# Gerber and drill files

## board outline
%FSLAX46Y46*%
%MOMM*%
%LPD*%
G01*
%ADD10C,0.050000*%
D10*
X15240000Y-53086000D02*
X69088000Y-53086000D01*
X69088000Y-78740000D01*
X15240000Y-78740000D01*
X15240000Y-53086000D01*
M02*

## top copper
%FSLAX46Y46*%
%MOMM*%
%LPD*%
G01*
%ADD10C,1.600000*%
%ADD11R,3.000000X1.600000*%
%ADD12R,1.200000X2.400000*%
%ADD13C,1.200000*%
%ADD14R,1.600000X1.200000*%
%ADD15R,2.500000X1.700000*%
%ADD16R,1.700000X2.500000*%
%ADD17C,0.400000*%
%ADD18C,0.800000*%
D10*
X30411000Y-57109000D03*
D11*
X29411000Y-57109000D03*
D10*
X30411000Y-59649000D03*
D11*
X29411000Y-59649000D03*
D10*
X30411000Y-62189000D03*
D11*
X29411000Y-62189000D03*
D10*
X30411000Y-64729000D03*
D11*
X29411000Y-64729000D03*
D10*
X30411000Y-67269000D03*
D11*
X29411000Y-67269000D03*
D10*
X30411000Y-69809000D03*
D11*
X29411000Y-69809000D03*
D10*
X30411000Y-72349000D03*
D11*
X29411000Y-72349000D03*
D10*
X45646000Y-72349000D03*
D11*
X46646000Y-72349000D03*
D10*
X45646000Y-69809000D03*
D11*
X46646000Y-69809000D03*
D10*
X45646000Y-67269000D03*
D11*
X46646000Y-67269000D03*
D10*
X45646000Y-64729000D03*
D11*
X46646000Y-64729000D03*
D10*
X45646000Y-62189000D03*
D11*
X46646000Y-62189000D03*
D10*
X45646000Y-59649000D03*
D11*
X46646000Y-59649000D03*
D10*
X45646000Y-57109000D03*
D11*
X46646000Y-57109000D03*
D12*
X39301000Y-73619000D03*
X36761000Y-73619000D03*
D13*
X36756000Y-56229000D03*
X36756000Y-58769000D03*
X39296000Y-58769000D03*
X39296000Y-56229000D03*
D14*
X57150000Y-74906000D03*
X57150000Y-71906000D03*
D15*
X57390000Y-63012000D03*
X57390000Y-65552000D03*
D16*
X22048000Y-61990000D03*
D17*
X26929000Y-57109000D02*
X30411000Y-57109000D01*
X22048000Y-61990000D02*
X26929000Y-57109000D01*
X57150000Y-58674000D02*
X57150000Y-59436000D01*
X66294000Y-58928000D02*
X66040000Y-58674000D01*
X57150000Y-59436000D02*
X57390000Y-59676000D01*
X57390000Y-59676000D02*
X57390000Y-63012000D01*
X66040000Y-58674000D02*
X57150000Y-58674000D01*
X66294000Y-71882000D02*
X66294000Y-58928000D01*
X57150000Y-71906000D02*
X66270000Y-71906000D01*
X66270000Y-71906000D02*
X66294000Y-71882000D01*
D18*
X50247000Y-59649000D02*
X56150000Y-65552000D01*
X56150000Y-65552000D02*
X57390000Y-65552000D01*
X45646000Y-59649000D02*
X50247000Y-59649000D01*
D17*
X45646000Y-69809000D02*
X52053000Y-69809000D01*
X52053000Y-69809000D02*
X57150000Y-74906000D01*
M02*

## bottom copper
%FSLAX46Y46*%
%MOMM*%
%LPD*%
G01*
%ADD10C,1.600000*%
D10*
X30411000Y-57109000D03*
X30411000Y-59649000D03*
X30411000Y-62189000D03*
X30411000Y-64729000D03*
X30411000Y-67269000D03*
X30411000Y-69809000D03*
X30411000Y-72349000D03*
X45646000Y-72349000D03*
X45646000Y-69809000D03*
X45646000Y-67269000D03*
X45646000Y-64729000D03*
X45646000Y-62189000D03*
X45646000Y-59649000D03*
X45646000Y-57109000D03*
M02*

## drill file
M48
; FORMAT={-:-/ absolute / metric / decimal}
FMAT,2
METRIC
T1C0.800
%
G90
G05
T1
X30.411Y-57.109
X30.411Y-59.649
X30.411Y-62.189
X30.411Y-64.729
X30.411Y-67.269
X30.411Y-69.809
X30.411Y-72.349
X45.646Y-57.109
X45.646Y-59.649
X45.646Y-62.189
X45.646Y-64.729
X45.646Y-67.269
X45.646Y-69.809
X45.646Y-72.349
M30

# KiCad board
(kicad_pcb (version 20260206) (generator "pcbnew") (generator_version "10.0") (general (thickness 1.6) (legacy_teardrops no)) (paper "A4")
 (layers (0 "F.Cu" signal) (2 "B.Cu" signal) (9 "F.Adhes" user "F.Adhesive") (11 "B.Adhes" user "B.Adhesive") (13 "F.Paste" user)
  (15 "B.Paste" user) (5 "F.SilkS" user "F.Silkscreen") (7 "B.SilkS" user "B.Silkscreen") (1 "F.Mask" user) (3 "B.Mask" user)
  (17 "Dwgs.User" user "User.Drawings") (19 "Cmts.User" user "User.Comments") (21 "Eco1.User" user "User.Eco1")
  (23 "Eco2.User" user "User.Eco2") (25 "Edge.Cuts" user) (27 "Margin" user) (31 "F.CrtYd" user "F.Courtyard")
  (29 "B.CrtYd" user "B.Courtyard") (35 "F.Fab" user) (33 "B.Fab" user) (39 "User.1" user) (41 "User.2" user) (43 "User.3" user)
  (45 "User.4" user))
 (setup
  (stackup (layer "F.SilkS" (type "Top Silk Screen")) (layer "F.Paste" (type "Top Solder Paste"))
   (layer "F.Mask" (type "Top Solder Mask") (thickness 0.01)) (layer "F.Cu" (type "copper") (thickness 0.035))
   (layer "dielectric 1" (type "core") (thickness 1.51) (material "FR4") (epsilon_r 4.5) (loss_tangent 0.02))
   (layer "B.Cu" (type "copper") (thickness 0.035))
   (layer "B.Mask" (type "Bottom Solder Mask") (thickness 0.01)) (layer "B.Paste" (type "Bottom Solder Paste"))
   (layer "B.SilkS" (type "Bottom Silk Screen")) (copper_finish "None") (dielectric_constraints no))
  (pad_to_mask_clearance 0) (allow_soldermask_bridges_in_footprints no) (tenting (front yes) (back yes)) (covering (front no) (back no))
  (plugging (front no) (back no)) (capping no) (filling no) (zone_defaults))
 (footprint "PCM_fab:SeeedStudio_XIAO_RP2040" (layer "F.Cu") (at 38.026 64.729)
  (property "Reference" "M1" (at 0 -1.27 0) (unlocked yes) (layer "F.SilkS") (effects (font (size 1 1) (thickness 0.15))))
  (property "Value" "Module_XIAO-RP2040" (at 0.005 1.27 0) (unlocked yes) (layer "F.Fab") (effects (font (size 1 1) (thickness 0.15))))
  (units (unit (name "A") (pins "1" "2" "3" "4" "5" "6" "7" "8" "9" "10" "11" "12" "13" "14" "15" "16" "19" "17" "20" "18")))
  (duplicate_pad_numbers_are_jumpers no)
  (pad "1" thru_hole circle (at -7.615 -7.62) (size 1.6 1.6) (drill 0.8) (layers "*.Cu" "*.Mask") (remove_unused_layers no) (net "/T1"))
  (pad "1" smd rect (at -7.615 -7.62) (size 3 1.6) (drill (offset -1 0)) (layers "F.Cu" "F.Mask" "F.Paste") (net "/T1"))
  (pad "2" thru_hole circle (at -7.615 -5.08) (size 1.6 1.6) (drill 0.8) (layers "*.Cu" "*.Mask") (remove_unused_layers no)
   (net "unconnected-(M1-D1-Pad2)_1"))
  (pad "2" smd rect (at -7.615 -5.08) (size 3 1.6) (drill (offset -1 0)) (layers "F.Cu" "F.Mask" "F.Paste") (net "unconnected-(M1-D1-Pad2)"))
  (pad "3" thru_hole circle (at -7.615 -2.54) (size 1.6 1.6) (drill 0.8) (layers "*.Cu" "*.Mask") (remove_unused_layers no)
   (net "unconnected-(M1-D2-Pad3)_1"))
  (pad "3" smd rect (at -7.615 -2.54) (size 3 1.6) (drill (offset -1 0)) (layers "F.Cu" "F.Mask" "F.Paste") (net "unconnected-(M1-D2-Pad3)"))
  (pad "4" thru_hole circle (at -7.615 0) (size 1.6 1.6) (drill 0.8) (layers "*.Cu" "*.Mask") (remove_unused_layers no)
   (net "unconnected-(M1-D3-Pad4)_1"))
  (pad "4" smd rect (at -7.615 0) (size 3 1.6) (drill (offset -1 0)) (layers "F.Cu" "F.Mask" "F.Paste") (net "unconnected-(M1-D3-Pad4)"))
  (pad "5" thru_hole circle (at -7.615 2.54) (size 1.6 1.6) (drill 0.8) (layers "*.Cu" "*.Mask") (remove_unused_layers no)
   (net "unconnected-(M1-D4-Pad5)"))
  (pad "5" smd rect (at -7.615 2.54) (size 3 1.6) (drill (offset -1 0)) (layers "F.Cu" "F.Mask" "F.Paste")
   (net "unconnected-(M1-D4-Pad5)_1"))
  (pad "6" thru_hole circle (at -7.615 5.08) (size 1.6 1.6) (drill 0.8) (layers "*.Cu" "*.Mask") (remove_unused_layers no)
   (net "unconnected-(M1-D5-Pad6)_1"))
  (pad "6" smd rect (at -7.615 5.08) (size 3 1.6) (drill (offset -1 0)) (layers "F.Cu" "F.Mask" "F.Paste") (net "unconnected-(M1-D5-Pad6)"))
  (pad "7" thru_hole circle (at -7.615 7.62) (size 1.6 1.6) (drill 0.8) (layers "*.Cu" "*.Mask") (remove_unused_layers no)
   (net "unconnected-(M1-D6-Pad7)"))
  (pad "7" smd rect (at -7.615 7.62) (size 3 1.6) (drill (offset -1 0)) (layers "F.Cu" "F.Mask" "F.Paste")
   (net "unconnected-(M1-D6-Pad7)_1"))
  (pad "8" thru_hole circle (at 7.62 7.62) (size 1.6 1.6) (drill 0.8) (layers "*.Cu" "*.Mask") (remove_unused_layers no)
   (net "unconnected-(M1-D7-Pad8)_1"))
  (pad "8" smd rect (at 7.62 7.62) (size 3 1.6) (drill (offset 1 0)) (layers "F.Cu" "F.Mask" "F.Paste") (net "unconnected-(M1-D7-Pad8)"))
  (pad "9" thru_hole circle (at 7.62 5.08) (size 1.6 1.6) (drill 0.8) (layers "*.Cu" "*.Mask") (remove_unused_layers no) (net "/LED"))
  (pad "9" smd rect (at 7.62 5.08) (size 3 1.6) (drill (offset 1 0)) (layers "F.Cu" "F.Mask" "F.Paste") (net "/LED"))
  (pad "10" thru_hole circle (at 7.62 2.54) (size 1.6 1.6) (drill 0.8) (layers "*.Cu" "*.Mask") (remove_unused_layers no) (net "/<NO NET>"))
  (pad "10" smd rect (at 7.62 2.54) (size 3 1.6) (drill (offset 1 0)) (layers "F.Cu" "F.Mask" "F.Paste") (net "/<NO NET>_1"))
  (pad "11" thru_hole circle (at 7.62 0) (size 1.6 1.6) (drill 0.8) (layers "*.Cu" "*.Mask") (remove_unused_layers no)
   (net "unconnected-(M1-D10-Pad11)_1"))
  (pad "11" smd rect (at 7.62 0) (size 3 1.6) (drill (offset 1 0)) (layers "F.Cu" "F.Mask" "F.Paste") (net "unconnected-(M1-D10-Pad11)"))
  (pad "12" thru_hole circle (at 7.62 -2.54) (size 1.6 1.6) (drill 0.8) (layers "*.Cu" "*.Mask") (remove_unused_layers no)
   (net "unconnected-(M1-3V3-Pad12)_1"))
  (pad "12" smd rect (at 7.62 -2.54) (size 3 1.6) (drill (offset 1 0)) (layers "F.Cu" "F.Mask" "F.Paste") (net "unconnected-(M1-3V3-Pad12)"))
  (pad "13" thru_hole circle (at 7.62 -5.08) (size 1.6 1.6) (drill 0.8) (layers "*.Cu" "*.Mask") (remove_unused_layers no) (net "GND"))
  (pad "13" smd rect (at 7.62 -5.08) (size 3 1.6) (drill (offset 1 0)) (layers "F.Cu" "F.Mask" "F.Paste") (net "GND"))
  (pad "14" thru_hole circle (at 7.62 -7.62) (size 1.6 1.6) (drill 0.8) (layers "*.Cu" "*.Mask") (remove_unused_layers no)
   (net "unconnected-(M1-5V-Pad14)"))
  (pad "14" smd rect (at 7.62 -7.62) (size 3 1.6) (drill (offset 1 0)) (layers "F.Cu" "F.Mask" "F.Paste")
   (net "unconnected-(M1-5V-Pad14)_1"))
  (pad "15" smd rect (at 1.275 8.89 270) (size 2.4 1.2) (layers "F.Cu" "F.Mask" "F.Paste") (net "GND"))
  (pad "16" smd rect (at -1.265 8.89 270) (size 2.4 1.2) (layers "F.Cu" "F.Mask" "F.Paste") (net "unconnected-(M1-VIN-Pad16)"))
  (pad "17" smd circle (at -1.27 -8.5) (size 1.2 1.2) (layers "F.Cu" "F.Mask" "F.Paste") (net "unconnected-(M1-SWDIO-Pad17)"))
  (pad "18" smd circle (at -1.27 -5.96) (size 1.2 1.2) (layers "F.Cu" "F.Mask" "F.Paste") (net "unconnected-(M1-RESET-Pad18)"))
  (pad "19" smd circle (at 1.27 -5.96) (size 1.2 1.2) (layers "F.Cu" "F.Mask" "F.Paste") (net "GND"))
  (pad "20" smd circle (at 1.27 -8.5) (size 1.2 1.2) (layers "F.Cu" "F.Mask" "F.Paste") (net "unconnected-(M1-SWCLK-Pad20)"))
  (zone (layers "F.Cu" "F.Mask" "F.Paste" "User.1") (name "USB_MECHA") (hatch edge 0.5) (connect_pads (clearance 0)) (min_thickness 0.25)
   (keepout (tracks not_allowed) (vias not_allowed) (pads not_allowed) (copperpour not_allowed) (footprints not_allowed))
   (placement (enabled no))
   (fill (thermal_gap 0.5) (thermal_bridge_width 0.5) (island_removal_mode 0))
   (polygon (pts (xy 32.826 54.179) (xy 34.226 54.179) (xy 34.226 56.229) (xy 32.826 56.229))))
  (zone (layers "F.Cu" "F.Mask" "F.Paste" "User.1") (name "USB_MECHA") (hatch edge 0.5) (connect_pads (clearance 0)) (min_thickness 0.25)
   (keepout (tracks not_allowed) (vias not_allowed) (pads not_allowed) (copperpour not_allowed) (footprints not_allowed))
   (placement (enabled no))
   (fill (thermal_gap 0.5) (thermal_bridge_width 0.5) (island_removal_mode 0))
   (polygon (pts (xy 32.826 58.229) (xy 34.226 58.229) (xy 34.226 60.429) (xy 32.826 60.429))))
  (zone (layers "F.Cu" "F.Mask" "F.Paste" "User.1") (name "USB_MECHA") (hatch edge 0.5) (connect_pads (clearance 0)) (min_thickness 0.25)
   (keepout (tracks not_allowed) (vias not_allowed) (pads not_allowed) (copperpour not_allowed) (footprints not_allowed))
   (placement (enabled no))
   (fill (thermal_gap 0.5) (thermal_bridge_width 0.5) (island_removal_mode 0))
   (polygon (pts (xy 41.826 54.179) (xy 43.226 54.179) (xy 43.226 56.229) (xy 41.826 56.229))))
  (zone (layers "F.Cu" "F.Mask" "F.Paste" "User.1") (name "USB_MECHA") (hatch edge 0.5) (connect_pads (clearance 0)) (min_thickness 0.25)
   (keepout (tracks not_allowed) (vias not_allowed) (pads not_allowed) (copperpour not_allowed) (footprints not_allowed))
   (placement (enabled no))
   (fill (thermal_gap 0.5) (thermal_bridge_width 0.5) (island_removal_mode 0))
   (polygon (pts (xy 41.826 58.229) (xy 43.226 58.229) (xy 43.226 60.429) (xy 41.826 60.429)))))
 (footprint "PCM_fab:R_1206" (layer "F.Cu") (at 57.15 73.406 90)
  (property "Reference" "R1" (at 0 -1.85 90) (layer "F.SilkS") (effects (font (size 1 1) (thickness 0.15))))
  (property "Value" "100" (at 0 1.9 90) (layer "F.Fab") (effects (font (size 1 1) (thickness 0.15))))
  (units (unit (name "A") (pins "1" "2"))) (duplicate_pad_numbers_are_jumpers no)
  (pad "1" smd rect (at -1.5 0 90) (size 1.2 1.6) (layers "F.Cu" "F.Mask" "F.Paste") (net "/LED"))
  (pad "2" smd rect (at 1.5 0 90) (size 1.2 1.6) (layers "F.Cu" "F.Mask" "F.Paste") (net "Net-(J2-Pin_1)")))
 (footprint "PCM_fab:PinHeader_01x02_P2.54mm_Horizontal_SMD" (layer "F.Cu") (at 57.39 63.012)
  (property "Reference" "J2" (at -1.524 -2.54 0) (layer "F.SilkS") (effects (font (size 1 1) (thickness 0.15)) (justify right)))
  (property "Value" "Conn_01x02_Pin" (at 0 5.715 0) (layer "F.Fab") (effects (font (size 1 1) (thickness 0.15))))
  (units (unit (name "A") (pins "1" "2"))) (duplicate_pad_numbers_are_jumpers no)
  (pad "1" smd rect (at 0 0) (size 2.5 1.7) (layers "F.Cu" "F.Mask" "F.Paste") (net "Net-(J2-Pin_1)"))
  (pad "2" smd rect (at 0 2.54) (size 2.5 1.7) (layers "F.Cu" "F.Mask" "F.Paste") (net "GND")))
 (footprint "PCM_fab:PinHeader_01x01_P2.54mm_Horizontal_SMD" (layer "F.Cu") (at 22.048 61.99 90)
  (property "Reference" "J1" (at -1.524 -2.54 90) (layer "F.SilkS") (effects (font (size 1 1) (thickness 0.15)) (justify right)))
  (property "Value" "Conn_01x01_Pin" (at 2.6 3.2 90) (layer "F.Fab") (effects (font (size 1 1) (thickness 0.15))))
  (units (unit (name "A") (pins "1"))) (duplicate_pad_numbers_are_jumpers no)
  (pad "1" smd rect (at 0 0 90) (size 2.5 1.7) (layers "F.Cu" "F.Mask" "F.Paste") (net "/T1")))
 (gr_rect (start 15.24 53.086) (end 69.088 78.74) (stroke (width 0.05) (type default)) (fill no) (layer "Edge.Cuts"))
 (segment (start 26.929 57.109) (end 30.411 57.109) (width 0.4) (layer "F.Cu") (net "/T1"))
 (segment (start 22.048 61.99) (end 26.929 57.109) (width 0.4) (layer "F.Cu") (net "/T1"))
 (segment (start 57.15 58.674) (end 57.15 59.436) (width 0.4) (layer "F.Cu") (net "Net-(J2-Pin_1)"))
 (segment (start 66.294 58.928) (end 66.04 58.674) (width 0.4) (layer "F.Cu") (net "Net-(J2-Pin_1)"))
 (segment (start 57.15 59.436) (end 57.39 59.676) (width 0.4) (layer "F.Cu") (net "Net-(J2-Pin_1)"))
 (segment (start 57.39 59.676) (end 57.39 63.012) (width 0.4) (layer "F.Cu") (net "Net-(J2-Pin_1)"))
 (segment (start 66.04 58.674) (end 57.15 58.674) (width 0.4) (layer "F.Cu") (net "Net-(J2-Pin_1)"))
 (segment (start 66.294 71.882) (end 66.294 58.928) (width 0.4) (layer "F.Cu") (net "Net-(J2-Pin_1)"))
 (segment (start 57.15 71.906) (end 66.27 71.906) (width 0.4) (layer "F.Cu") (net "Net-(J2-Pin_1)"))
 (segment (start 66.27 71.906) (end 66.294 71.882) (width 0.4) (layer "F.Cu") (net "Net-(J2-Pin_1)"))
 (segment (start 50.247 59.649) (end 56.15 65.552) (width 0.8) (layer "F.Cu") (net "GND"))
 (segment (start 56.15 65.552) (end 57.39 65.552) (width 0.8) (layer "F.Cu") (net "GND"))
 (segment (start 45.646 59.649) (end 50.247 59.649) (width 0.8) (layer "F.Cu") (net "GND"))
 (segment (start 45.646 69.809) (end 52.053 69.809) (width 0.4) (layer "F.Cu") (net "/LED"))
 (segment (start 52.053 69.809) (end 57.15 74.906) (width 0.4) (layer "F.Cu") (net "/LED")))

